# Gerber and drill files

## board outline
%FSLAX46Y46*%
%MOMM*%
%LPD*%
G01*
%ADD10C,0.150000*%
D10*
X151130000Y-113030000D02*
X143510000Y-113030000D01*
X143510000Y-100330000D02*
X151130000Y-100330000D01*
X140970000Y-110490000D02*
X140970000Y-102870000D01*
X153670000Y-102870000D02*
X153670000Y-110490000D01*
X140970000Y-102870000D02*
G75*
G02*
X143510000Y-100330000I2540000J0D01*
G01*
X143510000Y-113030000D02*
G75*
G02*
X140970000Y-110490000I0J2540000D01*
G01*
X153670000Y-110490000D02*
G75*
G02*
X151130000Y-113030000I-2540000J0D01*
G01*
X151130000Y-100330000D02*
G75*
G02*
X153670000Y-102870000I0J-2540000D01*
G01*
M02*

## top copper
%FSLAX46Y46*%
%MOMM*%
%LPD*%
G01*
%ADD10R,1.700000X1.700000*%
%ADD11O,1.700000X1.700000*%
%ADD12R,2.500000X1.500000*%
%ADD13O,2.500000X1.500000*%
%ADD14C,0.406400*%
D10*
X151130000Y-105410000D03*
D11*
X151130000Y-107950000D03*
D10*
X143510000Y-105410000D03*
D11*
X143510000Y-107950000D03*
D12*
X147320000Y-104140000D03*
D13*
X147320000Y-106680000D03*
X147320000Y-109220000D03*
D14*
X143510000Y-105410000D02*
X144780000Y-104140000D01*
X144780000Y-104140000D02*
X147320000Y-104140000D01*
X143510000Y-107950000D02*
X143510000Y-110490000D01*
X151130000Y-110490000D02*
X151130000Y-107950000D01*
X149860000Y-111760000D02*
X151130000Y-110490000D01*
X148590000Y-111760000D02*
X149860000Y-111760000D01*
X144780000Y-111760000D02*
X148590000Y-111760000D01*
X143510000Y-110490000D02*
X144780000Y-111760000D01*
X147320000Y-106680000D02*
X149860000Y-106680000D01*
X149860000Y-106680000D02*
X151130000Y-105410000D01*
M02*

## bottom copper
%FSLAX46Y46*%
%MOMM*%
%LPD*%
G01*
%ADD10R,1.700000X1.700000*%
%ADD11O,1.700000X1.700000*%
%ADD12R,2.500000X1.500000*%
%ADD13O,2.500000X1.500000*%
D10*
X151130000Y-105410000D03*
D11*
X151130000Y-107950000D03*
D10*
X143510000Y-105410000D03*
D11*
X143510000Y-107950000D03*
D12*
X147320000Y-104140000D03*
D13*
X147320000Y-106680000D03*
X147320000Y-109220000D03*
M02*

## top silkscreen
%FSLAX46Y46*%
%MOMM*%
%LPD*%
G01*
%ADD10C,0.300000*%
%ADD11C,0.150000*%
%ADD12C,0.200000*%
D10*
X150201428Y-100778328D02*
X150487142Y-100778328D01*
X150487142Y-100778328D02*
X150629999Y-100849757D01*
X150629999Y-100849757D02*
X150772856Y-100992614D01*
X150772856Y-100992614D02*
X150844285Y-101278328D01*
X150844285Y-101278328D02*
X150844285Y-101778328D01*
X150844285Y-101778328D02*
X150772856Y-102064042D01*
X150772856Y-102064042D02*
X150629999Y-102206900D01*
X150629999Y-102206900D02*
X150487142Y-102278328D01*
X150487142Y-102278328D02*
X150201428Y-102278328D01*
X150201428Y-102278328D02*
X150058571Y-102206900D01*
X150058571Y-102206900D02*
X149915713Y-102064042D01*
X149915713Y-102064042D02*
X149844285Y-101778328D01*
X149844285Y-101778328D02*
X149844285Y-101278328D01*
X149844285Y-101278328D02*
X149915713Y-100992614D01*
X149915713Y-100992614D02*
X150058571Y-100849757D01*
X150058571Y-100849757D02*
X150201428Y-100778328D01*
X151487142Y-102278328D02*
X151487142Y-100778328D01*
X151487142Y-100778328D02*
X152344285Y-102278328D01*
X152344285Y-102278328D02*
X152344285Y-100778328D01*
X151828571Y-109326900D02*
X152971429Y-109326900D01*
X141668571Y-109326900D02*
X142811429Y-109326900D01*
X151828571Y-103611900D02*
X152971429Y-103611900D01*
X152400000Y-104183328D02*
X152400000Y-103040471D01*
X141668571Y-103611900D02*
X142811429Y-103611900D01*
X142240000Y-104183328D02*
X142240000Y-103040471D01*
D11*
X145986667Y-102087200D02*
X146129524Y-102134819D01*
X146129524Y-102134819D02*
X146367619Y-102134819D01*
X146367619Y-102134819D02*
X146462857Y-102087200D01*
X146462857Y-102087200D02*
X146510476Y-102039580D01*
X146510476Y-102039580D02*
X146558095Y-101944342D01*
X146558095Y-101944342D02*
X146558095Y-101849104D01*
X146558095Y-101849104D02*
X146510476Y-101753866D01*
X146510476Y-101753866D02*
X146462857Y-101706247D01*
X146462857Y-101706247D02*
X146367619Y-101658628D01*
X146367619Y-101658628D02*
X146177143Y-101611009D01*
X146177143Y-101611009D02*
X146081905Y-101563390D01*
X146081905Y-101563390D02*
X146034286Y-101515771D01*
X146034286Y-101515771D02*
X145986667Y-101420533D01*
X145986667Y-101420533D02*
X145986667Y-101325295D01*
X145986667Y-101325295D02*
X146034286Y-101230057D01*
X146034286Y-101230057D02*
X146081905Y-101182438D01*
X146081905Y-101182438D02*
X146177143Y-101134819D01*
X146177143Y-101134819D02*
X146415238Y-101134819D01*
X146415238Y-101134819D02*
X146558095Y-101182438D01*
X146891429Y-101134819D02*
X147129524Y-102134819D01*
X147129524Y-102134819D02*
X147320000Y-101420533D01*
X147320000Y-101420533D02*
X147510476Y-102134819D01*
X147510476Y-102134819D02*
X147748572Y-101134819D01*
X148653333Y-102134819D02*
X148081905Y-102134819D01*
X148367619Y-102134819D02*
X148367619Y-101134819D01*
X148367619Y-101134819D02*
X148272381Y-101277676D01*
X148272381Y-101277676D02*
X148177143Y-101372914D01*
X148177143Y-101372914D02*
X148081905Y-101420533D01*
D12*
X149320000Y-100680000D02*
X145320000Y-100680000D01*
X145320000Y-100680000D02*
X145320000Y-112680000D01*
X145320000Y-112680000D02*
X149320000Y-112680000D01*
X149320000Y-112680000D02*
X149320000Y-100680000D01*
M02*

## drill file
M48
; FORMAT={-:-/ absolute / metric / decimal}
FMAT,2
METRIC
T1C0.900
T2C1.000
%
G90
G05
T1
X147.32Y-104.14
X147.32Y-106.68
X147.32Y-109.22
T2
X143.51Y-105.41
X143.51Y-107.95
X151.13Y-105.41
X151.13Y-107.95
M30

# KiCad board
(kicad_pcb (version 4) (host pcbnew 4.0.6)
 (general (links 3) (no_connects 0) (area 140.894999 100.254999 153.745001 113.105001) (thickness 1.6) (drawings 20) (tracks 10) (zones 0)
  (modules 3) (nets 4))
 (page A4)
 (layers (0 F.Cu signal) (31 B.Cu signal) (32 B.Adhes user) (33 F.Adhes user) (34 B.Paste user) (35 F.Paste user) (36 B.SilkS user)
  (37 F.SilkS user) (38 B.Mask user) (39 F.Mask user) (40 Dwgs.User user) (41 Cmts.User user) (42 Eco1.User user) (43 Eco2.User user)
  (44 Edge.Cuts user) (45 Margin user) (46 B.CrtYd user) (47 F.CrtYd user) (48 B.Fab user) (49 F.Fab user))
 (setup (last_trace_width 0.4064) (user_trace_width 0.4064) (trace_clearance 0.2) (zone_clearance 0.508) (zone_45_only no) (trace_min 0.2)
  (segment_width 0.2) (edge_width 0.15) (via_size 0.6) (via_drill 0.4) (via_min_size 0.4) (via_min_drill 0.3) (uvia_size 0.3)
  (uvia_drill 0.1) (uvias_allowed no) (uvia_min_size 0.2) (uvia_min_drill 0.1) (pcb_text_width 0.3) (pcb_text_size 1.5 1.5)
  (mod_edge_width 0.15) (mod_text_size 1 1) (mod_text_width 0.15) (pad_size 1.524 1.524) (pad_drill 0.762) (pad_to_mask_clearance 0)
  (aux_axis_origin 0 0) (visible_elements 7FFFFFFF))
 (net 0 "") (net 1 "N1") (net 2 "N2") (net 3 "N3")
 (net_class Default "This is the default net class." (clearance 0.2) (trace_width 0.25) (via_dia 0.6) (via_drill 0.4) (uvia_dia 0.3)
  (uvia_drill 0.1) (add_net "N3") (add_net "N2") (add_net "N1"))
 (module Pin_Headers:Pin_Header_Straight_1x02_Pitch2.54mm (layer F.Cu) (at 151.13 105.41)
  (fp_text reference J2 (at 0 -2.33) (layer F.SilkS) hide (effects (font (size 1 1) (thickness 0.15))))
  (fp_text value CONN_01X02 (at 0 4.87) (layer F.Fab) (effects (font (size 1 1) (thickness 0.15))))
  (pad 1 thru_hole rect (at 0 0) (size 1.7 1.7) (drill 1) (layers *.Cu *.Mask) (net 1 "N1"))
  (pad 2 thru_hole oval (at 0 2.54) (size 1.7 1.7) (drill 1) (layers *.Cu *.Mask) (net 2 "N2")))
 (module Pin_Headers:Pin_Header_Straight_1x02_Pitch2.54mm (layer F.Cu) (at 143.51 105.41)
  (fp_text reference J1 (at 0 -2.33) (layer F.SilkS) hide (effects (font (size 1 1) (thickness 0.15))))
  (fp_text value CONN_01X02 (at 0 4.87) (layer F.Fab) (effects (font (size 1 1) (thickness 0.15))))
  (pad 1 thru_hole rect (at 0 0) (size 1.7 1.7) (drill 1) (layers *.Cu *.Mask) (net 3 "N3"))
  (pad 2 thru_hole oval (at 0 2.54) (size 1.7 1.7) (drill 1) (layers *.Cu *.Mask) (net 2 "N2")))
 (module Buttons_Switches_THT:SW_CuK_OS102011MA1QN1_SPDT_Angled (layer F.Cu) (at 147.32 106.68 270)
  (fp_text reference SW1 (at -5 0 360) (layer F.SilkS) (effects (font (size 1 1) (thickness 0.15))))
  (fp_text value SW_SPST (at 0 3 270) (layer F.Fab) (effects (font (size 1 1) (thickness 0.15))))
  (fp_line (start -6 -2) (end -6 2) (layer F.SilkS) (width 0.2)) (fp_line (start -6 2) (end 6 2) (layer F.SilkS) (width 0.2))
  (fp_line (start 6 2) (end 6 -2) (layer F.SilkS) (width 0.2))
  (fp_line (start 6 -2) (end -6 -2) (layer F.SilkS) (width 0.2))
  (pad 1 thru_hole rect (at -2.54 0 270) (size 1.5 2.5) (drill 0.9) (layers *.Cu *.Mask) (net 3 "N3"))
  (pad 2 thru_hole oval (at 0 0 270) (size 1.5 2.5) (drill 0.9) (layers *.Cu *.Mask) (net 1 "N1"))
  (pad 3 thru_hole oval (at 2.54 0 270) (size 1.5 2.5) (drill 0.9) (layers *.Cu *.Mask)))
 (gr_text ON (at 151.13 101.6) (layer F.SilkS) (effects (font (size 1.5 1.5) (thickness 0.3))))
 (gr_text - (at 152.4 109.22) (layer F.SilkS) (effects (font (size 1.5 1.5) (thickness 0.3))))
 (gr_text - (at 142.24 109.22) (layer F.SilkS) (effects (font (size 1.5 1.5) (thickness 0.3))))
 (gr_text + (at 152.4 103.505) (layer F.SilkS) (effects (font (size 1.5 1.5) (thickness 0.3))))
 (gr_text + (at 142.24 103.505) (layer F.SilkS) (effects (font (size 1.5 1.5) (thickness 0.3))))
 (gr_line (start 151.13 113.03) (end 143.51 113.03) (angle 90) (layer Edge.Cuts) (width 0.15))
 (gr_line (start 143.51 100.33) (end 151.13 100.33) (angle 90) (layer Edge.Cuts) (width 0.15))
 (gr_line (start 140.97 110.49) (end 140.97 102.87) (angle 90) (layer Edge.Cuts) (width 0.15))
 (gr_line (start 153.67 102.87) (end 153.67 110.49) (angle 90) (layer Edge.Cuts) (width 0.15))
 (gr_arc (start 143.51 102.87) (end 140.97 102.87) (angle 90) (layer Edge.Cuts) (width 0.15))
 (gr_arc (start 143.51 110.49) (end 143.51 113.03) (angle 90) (layer Edge.Cuts) (width 0.15))
 (gr_arc (start 151.13 110.49) (end 153.67 110.49) (angle 90) (layer Edge.Cuts) (width 0.15))
 (gr_arc (start 151.13 102.87) (end 151.13 100.33) (angle 90) (layer Edge.Cuts) (width 0.15))
 (segment (start 143.51 105.41) (end 144.78 104.14) (width 0.4064) (layer F.Cu) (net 3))
 (segment (start 144.78 104.14) (end 147.32 104.14) (width 0.4064) (layer F.Cu) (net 3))
 (segment (start 143.51 107.95) (end 143.51 110.49) (width 0.4064) (layer F.Cu) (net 2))
 (segment (start 151.13 110.49) (end 151.13 107.95) (width 0.4064) (layer F.Cu) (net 2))
 (segment (start 149.86 111.76) (end 151.13 110.49) (width 0.4064) (layer F.Cu) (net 2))
 (segment (start 148.59 111.76) (end 149.86 111.76) (width 0.4064) (layer F.Cu) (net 2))
 (segment (start 144.78 111.76) (end 148.59 111.76) (width 0.4064) (layer F.Cu) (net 2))
 (segment (start 143.51 110.49) (end 144.78 111.76) (width 0.4064) (layer F.Cu) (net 2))
 (segment (start 147.32 106.68) (end 149.86 106.68) (width 0.4064) (layer F.Cu) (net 1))
 (segment (start 149.86 106.68) (end 151.13 105.41) (width 0.4064) (layer F.Cu) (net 1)))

